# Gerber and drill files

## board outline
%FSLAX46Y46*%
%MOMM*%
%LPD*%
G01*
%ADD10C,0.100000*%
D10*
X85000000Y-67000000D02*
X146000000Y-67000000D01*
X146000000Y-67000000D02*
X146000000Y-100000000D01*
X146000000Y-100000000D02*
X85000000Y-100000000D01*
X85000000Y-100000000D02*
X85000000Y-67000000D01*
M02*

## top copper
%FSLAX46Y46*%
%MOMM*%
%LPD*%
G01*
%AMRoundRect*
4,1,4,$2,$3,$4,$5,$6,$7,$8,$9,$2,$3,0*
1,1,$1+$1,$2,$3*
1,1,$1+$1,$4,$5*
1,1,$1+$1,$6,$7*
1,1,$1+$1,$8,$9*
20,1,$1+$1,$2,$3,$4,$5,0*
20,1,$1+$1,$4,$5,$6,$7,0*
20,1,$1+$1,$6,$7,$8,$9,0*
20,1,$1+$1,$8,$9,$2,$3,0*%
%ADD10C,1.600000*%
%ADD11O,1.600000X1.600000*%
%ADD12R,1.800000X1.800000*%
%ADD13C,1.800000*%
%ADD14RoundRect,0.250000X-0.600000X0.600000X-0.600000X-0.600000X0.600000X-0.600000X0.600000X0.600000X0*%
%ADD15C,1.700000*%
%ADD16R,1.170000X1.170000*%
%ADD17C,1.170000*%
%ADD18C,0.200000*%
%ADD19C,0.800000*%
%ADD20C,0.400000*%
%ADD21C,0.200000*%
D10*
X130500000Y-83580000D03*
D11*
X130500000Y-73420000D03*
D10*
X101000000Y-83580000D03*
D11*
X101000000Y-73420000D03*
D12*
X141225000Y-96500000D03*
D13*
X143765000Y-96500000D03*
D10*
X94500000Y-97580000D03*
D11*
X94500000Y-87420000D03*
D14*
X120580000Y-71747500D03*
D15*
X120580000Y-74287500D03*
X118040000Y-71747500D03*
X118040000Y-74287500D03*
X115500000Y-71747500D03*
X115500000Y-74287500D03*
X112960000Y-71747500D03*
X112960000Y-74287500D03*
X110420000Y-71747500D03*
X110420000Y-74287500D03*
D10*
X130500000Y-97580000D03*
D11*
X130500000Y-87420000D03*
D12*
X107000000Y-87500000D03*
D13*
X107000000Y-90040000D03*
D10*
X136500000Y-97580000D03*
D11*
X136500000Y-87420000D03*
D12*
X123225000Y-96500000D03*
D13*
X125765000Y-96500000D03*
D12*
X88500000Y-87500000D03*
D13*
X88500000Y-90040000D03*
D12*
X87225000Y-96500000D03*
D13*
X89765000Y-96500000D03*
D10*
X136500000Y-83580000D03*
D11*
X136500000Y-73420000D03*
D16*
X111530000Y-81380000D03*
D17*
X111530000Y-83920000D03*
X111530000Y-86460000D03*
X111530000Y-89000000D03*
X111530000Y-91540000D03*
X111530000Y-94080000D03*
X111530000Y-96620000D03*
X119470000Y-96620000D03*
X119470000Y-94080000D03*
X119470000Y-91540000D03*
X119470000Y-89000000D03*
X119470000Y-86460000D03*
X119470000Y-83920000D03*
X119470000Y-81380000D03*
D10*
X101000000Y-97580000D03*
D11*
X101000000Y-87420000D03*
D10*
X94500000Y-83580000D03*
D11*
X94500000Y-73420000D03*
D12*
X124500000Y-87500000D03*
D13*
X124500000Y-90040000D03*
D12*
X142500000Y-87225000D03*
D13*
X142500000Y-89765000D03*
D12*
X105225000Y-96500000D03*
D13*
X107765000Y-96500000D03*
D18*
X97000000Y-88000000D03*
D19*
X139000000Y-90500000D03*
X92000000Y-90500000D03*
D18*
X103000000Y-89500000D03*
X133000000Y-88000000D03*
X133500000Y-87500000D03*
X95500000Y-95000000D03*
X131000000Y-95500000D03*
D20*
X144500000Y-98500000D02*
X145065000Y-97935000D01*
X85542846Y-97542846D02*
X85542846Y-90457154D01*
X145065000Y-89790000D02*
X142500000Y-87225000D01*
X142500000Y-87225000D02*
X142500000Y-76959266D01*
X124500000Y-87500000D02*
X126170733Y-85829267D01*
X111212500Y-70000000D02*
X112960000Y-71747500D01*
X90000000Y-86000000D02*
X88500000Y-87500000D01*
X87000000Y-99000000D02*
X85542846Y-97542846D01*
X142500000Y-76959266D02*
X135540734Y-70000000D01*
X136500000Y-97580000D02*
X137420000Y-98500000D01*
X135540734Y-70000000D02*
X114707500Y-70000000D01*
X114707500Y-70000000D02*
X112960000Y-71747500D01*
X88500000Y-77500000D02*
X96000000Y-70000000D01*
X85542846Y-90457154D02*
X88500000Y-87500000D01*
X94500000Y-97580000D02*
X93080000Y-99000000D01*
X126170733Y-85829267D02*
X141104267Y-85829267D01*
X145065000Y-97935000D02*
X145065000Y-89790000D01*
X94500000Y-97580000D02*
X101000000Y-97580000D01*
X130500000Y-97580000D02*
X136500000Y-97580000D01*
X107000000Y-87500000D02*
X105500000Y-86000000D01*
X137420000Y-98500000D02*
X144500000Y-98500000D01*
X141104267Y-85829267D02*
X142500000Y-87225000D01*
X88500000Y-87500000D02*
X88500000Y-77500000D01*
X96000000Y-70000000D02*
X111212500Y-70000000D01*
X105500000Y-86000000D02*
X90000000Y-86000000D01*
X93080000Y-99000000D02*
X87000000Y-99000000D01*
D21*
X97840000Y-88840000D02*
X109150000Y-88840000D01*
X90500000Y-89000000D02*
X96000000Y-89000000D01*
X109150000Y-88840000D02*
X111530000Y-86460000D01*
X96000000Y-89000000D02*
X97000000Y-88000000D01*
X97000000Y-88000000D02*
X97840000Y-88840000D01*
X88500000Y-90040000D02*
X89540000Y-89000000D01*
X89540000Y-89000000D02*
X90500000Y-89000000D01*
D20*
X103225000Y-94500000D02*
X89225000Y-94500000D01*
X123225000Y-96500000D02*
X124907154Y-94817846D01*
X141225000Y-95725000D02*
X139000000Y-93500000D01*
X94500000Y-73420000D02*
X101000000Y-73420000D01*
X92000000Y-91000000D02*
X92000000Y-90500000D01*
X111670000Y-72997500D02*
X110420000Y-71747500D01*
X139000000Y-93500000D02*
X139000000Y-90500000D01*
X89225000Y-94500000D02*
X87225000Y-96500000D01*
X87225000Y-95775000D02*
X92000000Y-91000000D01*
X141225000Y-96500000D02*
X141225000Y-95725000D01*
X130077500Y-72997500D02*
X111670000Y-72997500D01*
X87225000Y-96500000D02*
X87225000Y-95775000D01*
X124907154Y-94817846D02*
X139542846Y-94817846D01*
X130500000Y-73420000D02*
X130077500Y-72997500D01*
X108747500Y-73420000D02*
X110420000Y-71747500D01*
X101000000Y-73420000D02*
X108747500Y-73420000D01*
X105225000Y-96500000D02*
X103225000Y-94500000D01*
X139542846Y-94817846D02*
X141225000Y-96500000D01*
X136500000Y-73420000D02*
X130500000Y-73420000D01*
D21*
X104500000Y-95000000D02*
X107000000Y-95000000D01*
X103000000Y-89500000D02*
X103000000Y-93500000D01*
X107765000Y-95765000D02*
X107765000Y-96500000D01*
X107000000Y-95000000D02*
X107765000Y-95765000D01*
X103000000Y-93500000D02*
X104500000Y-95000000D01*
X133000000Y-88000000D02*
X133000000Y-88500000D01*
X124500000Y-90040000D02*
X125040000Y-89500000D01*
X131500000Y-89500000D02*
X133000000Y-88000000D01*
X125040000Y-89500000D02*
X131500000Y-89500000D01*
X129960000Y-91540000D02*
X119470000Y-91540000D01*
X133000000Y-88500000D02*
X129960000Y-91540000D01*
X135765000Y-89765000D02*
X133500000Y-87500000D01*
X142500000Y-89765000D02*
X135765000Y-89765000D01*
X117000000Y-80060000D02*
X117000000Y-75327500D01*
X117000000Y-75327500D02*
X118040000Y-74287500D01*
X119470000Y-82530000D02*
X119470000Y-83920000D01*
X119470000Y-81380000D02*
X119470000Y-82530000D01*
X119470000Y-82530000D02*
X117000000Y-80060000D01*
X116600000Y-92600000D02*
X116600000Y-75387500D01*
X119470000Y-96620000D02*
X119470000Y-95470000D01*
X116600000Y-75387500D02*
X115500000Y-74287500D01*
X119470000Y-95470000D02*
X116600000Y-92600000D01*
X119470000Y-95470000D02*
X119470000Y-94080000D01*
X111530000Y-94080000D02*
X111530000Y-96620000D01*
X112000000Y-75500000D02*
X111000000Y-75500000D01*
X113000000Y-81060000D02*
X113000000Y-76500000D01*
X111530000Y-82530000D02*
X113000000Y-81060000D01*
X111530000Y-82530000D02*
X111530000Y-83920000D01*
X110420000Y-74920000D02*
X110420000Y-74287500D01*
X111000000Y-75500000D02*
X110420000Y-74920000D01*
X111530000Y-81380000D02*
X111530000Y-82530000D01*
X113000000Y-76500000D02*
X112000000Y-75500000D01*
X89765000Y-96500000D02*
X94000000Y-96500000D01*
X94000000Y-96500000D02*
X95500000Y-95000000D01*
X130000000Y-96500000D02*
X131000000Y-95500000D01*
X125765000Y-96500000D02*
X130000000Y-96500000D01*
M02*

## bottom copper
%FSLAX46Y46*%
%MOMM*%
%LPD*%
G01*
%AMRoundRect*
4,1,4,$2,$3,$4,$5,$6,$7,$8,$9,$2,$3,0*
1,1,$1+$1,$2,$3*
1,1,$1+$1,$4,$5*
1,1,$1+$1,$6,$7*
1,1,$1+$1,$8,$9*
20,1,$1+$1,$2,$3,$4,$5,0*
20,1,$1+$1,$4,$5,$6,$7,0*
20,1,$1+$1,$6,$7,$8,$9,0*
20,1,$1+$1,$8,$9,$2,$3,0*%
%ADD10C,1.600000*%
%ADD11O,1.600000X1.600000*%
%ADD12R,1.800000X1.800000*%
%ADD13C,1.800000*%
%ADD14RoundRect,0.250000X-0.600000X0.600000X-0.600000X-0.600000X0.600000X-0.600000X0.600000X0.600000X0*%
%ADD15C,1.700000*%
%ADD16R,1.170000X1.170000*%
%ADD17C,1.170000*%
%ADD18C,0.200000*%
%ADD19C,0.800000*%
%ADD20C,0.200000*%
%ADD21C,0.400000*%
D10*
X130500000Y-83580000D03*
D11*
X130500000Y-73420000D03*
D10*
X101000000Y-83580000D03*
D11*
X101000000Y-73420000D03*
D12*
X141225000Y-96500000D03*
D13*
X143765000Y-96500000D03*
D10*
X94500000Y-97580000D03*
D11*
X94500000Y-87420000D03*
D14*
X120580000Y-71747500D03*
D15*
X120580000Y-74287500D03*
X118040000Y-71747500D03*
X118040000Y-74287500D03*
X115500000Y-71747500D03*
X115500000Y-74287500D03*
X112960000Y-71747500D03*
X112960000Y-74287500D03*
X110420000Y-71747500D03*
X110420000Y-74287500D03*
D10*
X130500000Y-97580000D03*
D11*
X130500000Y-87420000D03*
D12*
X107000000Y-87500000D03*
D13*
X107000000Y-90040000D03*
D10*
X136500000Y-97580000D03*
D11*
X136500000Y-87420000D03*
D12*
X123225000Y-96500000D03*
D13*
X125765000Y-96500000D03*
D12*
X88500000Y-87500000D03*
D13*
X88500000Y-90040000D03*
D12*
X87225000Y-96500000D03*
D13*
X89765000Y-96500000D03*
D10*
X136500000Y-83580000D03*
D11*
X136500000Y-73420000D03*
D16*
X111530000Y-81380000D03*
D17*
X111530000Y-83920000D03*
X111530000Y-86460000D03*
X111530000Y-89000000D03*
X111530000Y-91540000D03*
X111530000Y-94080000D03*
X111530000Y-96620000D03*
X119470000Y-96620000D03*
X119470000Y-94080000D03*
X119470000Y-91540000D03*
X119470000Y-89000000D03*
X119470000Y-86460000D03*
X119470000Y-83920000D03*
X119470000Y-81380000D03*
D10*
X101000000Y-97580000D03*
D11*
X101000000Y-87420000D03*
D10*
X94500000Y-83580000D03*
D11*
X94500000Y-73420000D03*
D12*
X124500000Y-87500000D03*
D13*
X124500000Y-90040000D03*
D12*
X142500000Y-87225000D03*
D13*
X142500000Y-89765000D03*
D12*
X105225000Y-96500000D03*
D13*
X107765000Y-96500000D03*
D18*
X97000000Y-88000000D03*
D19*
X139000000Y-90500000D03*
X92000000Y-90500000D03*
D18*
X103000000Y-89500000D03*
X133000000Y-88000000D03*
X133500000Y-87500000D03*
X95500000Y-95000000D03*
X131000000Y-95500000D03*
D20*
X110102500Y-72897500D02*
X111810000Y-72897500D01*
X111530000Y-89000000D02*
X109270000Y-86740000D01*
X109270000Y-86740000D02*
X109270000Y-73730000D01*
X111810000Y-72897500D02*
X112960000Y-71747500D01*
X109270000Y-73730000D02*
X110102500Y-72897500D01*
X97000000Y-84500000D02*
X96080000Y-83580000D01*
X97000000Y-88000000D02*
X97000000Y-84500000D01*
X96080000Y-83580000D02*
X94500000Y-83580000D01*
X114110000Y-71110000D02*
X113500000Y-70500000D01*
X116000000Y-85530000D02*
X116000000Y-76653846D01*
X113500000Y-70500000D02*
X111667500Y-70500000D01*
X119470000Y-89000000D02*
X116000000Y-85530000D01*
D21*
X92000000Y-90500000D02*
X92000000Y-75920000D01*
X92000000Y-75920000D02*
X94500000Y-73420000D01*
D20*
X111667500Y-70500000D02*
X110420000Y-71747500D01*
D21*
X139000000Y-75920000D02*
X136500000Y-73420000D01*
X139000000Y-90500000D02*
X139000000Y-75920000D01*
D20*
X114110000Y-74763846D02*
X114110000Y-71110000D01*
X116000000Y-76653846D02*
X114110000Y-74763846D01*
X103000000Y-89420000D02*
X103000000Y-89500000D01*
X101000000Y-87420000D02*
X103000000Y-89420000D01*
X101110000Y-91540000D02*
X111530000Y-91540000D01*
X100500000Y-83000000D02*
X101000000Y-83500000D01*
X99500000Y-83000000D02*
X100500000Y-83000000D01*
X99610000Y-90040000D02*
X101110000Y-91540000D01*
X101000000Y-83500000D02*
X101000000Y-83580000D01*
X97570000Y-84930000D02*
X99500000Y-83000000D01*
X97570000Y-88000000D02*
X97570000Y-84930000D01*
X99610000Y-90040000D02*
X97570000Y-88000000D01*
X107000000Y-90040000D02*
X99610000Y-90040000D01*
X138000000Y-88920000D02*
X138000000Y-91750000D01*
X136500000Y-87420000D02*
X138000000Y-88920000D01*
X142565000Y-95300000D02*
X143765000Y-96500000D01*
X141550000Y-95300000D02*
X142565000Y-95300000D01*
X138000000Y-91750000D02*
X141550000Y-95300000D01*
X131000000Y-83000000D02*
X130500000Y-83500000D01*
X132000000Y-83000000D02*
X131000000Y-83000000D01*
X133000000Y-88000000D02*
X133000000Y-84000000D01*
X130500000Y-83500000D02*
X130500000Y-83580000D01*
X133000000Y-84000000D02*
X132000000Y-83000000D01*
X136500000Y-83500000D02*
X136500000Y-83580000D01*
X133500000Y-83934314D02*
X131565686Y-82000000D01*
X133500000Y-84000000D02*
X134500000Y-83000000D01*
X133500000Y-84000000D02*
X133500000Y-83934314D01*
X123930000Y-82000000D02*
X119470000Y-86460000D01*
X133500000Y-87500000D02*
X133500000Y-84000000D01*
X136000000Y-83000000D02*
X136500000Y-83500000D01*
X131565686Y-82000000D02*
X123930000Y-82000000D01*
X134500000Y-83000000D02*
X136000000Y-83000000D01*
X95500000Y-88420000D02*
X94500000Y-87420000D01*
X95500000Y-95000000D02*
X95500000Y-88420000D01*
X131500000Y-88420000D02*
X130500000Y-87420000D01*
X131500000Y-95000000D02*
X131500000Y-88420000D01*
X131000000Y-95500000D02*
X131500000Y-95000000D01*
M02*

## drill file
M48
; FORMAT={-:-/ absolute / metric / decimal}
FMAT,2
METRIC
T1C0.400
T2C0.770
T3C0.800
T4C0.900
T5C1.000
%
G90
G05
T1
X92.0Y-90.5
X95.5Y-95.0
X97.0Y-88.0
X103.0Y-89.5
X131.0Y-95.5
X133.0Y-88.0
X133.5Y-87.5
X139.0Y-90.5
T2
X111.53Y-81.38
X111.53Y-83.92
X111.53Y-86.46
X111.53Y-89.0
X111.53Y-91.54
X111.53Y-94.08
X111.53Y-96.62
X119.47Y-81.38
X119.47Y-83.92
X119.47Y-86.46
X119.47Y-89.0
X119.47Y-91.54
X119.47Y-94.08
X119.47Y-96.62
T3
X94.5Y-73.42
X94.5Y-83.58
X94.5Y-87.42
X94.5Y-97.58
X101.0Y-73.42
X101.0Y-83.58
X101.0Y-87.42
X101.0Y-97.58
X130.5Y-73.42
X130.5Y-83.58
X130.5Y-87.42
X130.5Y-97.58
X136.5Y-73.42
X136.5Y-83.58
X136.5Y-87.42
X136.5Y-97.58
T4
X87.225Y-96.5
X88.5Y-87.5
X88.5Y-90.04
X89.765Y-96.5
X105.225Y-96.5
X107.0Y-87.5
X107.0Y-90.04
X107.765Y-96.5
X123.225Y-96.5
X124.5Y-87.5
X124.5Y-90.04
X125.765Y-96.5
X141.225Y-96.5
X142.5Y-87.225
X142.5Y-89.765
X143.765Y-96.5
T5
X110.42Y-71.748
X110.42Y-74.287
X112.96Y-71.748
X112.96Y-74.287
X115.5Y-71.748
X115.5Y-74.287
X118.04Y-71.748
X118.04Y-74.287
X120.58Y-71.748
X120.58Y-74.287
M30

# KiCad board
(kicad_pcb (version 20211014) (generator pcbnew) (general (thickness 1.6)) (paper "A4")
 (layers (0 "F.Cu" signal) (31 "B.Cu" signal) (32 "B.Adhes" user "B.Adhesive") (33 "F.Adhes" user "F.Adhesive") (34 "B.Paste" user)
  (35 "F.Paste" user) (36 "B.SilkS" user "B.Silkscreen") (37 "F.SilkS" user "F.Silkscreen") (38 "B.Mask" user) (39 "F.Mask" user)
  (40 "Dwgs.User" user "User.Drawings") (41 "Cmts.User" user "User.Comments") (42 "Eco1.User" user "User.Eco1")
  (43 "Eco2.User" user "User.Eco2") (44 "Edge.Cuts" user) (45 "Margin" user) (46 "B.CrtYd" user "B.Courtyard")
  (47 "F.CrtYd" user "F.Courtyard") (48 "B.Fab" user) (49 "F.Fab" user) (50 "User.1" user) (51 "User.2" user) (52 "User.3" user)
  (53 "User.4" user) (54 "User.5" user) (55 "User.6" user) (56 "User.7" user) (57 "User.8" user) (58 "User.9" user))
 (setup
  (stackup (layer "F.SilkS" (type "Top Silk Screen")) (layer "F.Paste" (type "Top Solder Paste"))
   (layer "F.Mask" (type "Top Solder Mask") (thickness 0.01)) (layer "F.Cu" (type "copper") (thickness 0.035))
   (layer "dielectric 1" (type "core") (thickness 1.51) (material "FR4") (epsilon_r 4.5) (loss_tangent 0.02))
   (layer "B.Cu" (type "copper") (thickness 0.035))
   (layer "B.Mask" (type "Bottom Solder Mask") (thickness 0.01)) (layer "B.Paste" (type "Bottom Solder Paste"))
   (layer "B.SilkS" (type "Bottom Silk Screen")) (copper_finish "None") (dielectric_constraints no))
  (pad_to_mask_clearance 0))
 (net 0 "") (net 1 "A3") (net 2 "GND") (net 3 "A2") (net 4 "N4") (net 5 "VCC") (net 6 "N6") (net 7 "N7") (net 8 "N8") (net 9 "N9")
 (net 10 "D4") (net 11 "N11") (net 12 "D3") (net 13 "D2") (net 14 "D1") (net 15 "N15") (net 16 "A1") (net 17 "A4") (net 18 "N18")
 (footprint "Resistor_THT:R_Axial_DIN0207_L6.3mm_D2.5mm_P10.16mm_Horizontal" (layer "F.Cu") (at 130.5 83.58 90)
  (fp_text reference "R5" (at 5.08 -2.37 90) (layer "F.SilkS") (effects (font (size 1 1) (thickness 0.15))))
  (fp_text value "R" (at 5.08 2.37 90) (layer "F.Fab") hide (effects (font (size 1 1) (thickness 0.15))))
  (pad "1" thru_hole circle (at 0 0 90) (size 1.6 1.6) (drill 0.8) (layers *.Cu *.Mask) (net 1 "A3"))
  (pad "2" thru_hole oval (at 10.16 0 90) (size 1.6 1.6) (drill 0.8) (layers *.Cu *.Mask) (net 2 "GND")))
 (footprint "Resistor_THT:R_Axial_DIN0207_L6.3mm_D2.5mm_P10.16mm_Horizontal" (layer "F.Cu") (at 101 83.58 90)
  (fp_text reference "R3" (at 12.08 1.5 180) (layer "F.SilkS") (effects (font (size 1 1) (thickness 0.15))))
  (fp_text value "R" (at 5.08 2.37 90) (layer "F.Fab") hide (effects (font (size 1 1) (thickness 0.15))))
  (pad "1" thru_hole circle (at 0 0 90) (size 1.6 1.6) (drill 0.8) (layers *.Cu *.Mask) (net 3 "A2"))
  (pad "2" thru_hole oval (at 10.16 0 90) (size 1.6 1.6) (drill 0.8) (layers *.Cu *.Mask) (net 2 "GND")))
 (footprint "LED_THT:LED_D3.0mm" (layer "F.Cu") (at 141.225 96.5)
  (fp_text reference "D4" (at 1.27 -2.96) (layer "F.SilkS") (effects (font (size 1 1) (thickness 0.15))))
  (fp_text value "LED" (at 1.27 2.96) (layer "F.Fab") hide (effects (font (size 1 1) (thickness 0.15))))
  (pad "1" thru_hole rect (at 0 0) (size 1.8 1.8) (drill 0.9) (layers *.Cu *.Mask) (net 2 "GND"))
  (pad "2" thru_hole circle (at 2.54 0) (size 1.8 1.8) (drill 0.9) (layers *.Cu *.Mask) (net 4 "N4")))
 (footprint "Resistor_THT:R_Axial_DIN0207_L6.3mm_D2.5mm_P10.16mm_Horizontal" (layer "F.Cu") (at 94.5 97.58 90)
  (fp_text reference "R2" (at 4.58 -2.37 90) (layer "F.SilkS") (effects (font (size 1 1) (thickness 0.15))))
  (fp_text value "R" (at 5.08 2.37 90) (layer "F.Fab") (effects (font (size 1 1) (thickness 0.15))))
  (pad "1" thru_hole circle (at 0 0 90) (size 1.6 1.6) (drill 0.8) (layers *.Cu *.Mask) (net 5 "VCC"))
  (pad "2" thru_hole oval (at 10.16 0 90) (size 1.6 1.6) (drill 0.8) (layers *.Cu *.Mask) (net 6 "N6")))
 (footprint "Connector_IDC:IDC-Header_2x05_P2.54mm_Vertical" (layer "F.Cu") (at 120.58 71.7475 -90)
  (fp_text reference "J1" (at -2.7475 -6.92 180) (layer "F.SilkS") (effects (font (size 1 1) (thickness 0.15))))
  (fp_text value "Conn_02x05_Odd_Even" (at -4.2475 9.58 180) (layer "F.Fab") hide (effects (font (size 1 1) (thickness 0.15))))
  (pad "1" thru_hole roundrect (at 0 0 270) (size 1.7 1.7) (drill 1) (layers *.Cu *.Mask) (roundrect_rratio 0.147059) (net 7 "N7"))
  (pad "2" thru_hole circle (at 2.54 0 270) (size 1.7 1.7) (drill 1) (layers *.Cu *.Mask) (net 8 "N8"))
  (pad "3" thru_hole circle (at 0 2.54 270) (size 1.7 1.7) (drill 1) (layers *.Cu *.Mask) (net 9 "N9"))
  (pad "4" thru_hole circle (at 2.54 2.54 270) (size 1.7 1.7) (drill 1) (layers *.Cu *.Mask) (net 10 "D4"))
  (pad "5" thru_hole circle (at 0 5.08 270) (size 1.7 1.7) (drill 1) (layers *.Cu *.Mask) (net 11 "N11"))
  (pad "6" thru_hole circle (at 2.54 5.08 270) (size 1.7 1.7) (drill 1) (layers *.Cu *.Mask) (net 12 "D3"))
  (pad "7" thru_hole circle (at 0 7.62 270) (size 1.7 1.7) (drill 1) (layers *.Cu *.Mask) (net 5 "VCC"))
  (pad "8" thru_hole circle (at 2.54 7.62 270) (size 1.7 1.7) (drill 1) (layers *.Cu *.Mask) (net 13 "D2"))
  (pad "9" thru_hole circle (at 0 10.16 270) (size 1.7 1.7) (drill 1) (layers *.Cu *.Mask) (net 2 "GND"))
  (pad "10" thru_hole circle (at 2.54 10.16 270) (size 1.7 1.7) (drill 1) (layers *.Cu *.Mask) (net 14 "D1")))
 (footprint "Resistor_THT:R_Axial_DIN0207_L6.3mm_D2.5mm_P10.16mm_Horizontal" (layer "F.Cu") (at 130.5 97.58 90)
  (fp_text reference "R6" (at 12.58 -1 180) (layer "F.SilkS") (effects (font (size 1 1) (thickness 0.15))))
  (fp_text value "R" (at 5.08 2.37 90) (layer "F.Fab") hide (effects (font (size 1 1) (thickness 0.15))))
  (pad "1" thru_hole circle (at 0 0 90) (size 1.6 1.6) (drill 0.8) (layers *.Cu *.Mask) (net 5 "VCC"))
  (pad "2" thru_hole oval (at 10.16 0 90) (size 1.6 1.6) (drill 0.8) (layers *.Cu *.Mask) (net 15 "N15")))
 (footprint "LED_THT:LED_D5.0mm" (layer "F.Cu") (at 107 87.5 -90)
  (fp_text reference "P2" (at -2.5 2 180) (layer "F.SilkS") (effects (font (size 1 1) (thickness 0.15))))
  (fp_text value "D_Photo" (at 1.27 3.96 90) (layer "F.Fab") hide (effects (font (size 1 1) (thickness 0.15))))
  (pad "1" thru_hole rect (at 0 0 270) (size 1.8 1.8) (drill 0.9) (layers *.Cu *.Mask) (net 5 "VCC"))
  (pad "2" thru_hole circle (at 2.54 0 270) (size 1.8 1.8) (drill 0.9) (layers *.Cu *.Mask) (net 3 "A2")))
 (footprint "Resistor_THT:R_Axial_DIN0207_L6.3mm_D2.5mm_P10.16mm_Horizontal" (layer "F.Cu") (at 136.5 97.58 90)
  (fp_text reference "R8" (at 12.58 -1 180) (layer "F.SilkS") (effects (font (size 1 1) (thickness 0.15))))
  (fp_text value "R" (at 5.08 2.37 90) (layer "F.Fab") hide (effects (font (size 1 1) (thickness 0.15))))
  (pad "1" thru_hole circle (at 0 0 90) (size 1.6 1.6) (drill 0.8) (layers *.Cu *.Mask) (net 5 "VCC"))
  (pad "2" thru_hole oval (at 10.16 0 90) (size 1.6 1.6) (drill 0.8) (layers *.Cu *.Mask) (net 4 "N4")))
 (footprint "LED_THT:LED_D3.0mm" (layer "F.Cu") (at 123.225 96.5)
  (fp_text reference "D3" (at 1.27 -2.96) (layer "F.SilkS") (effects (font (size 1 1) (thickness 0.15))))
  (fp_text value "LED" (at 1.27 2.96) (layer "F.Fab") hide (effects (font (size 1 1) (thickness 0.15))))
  (pad "1" thru_hole rect (at 0 0) (size 1.8 1.8) (drill 0.9) (layers *.Cu *.Mask) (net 2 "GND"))
  (pad "2" thru_hole circle (at 2.54 0) (size 1.8 1.8) (drill 0.9) (layers *.Cu *.Mask) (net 15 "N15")))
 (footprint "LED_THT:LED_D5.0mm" (layer "F.Cu") (at 88.5 87.5 -90)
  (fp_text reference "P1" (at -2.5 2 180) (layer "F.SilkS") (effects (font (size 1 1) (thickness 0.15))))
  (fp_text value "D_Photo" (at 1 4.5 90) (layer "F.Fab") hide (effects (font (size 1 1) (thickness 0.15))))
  (pad "1" thru_hole rect (at 0 0 270) (size 1.8 1.8) (drill 0.9) (layers *.Cu *.Mask) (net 5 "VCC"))
  (pad "2" thru_hole circle (at 2.54 0 270) (size 1.8 1.8) (drill 0.9) (layers *.Cu *.Mask) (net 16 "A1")))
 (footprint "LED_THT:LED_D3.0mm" (layer "F.Cu") (at 87.225 96.5)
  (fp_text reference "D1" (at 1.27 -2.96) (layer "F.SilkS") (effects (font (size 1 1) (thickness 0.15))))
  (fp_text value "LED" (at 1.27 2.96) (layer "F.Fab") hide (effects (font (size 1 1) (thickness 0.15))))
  (pad "1" thru_hole rect (at 0 0) (size 1.8 1.8) (drill 0.9) (layers *.Cu *.Mask) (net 2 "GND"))
  (pad "2" thru_hole circle (at 2.54 0) (size 1.8 1.8) (drill 0.9) (layers *.Cu *.Mask) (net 6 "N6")))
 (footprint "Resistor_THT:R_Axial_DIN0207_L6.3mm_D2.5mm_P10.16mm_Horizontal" (layer "F.Cu") (at 136.5 83.58 90)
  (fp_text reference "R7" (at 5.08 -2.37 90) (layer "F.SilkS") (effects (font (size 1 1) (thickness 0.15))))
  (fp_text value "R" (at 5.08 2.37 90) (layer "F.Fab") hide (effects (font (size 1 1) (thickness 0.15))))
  (pad "1" thru_hole circle (at 0 0 90) (size 1.6 1.6) (drill 0.8) (layers *.Cu *.Mask) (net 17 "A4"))
  (pad "2" thru_hole oval (at 10.16 0 90) (size 1.6 1.6) (drill 0.8) (layers *.Cu *.Mask) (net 2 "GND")))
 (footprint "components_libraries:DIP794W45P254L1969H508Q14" (layer "F.Cu") (at 115.5 89)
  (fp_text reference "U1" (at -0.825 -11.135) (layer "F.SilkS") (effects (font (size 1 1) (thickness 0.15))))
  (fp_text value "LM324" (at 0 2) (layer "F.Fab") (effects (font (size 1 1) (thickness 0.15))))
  (pad "1" thru_hole rect locked (at -3.97 -7.62) (size 1.17 1.17) (drill 0.77) (layers *.Cu *.Mask) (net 14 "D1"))
  (pad "2" thru_hole circle locked (at -3.97 -5.08) (size 1.17 1.17) (drill 0.77) (layers *.Cu *.Mask) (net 14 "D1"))
  (pad "3" thru_hole circle locked (at -3.97 -2.54) (size 1.17 1.17) (drill 0.77) (layers *.Cu *.Mask) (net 16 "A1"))
  (pad "4" thru_hole circle locked (at -3.97 0) (size 1.17 1.17) (drill 0.77) (layers *.Cu *.Mask) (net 5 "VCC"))
  (pad "5" thru_hole circle locked (at -3.97 2.54) (size 1.17 1.17) (drill 0.77) (layers *.Cu *.Mask) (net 3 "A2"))
  (pad "6" thru_hole circle locked (at -3.97 5.08) (size 1.17 1.17) (drill 0.77) (layers *.Cu *.Mask) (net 13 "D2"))
  (pad "7" thru_hole circle locked (at -3.97 7.62) (size 1.17 1.17) (drill 0.77) (layers *.Cu *.Mask) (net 13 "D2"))
  (pad "8" thru_hole circle locked (at 3.97 7.62) (size 1.17 1.17) (drill 0.77) (layers *.Cu *.Mask) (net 12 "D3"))
  (pad "9" thru_hole circle locked (at 3.97 5.08) (size 1.17 1.17) (drill 0.77) (layers *.Cu *.Mask) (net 12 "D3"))
  (pad "10" thru_hole circle locked (at 3.97 2.54) (size 1.17 1.17) (drill 0.77) (layers *.Cu *.Mask) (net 1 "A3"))
  (pad "11" thru_hole circle locked (at 3.97 0) (size 1.17 1.17) (drill 0.77) (layers *.Cu *.Mask) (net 2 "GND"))
  (pad "12" thru_hole circle locked (at 3.97 -2.54) (size 1.17 1.17) (drill 0.77) (layers *.Cu *.Mask) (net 17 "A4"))
  (pad "13" thru_hole circle locked (at 3.97 -5.08) (size 1.17 1.17) (drill 0.77) (layers *.Cu *.Mask) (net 10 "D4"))
  (pad "14" thru_hole circle locked (at 3.97 -7.62) (size 1.17 1.17) (drill 0.77) (layers *.Cu *.Mask) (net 10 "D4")))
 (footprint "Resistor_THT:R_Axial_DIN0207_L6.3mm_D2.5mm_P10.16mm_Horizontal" (layer "F.Cu") (at 101 97.58 90)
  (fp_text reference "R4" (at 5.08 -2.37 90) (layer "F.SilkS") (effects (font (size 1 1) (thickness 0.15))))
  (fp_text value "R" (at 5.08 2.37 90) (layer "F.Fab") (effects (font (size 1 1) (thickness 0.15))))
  (pad "1" thru_hole circle (at 0 0 90) (size 1.6 1.6) (drill 0.8) (layers *.Cu *.Mask) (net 5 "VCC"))
  (pad "2" thru_hole oval (at 10.16 0 90) (size 1.6 1.6) (drill 0.8) (layers *.Cu *.Mask) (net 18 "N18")))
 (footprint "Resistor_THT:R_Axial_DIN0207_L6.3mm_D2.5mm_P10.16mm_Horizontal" (layer "F.Cu") (at 94.5 83.58 90)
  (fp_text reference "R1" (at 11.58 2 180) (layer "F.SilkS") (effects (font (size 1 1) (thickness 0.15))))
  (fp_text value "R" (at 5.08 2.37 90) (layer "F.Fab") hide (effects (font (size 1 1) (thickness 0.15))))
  (pad "1" thru_hole circle (at 0 0 90) (size 1.6 1.6) (drill 0.8) (layers *.Cu *.Mask) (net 16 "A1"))
  (pad "2" thru_hole oval (at 10.16 0 90) (size 1.6 1.6) (drill 0.8) (layers *.Cu *.Mask) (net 2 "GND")))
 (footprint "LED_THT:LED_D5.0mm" (layer "F.Cu") (at 124.5 87.5 -90)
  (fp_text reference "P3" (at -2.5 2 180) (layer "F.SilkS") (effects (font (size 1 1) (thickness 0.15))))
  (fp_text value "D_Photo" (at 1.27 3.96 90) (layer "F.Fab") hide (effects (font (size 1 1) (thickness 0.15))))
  (pad "1" thru_hole rect (at 0 0 270) (size 1.8 1.8) (drill 0.9) (layers *.Cu *.Mask) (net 5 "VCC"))
  (pad "2" thru_hole circle (at 2.54 0 270) (size 1.8 1.8) (drill 0.9) (layers *.Cu *.Mask) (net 1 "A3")))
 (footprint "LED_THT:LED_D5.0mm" (layer "F.Cu") (at 142.5 87.225 -90)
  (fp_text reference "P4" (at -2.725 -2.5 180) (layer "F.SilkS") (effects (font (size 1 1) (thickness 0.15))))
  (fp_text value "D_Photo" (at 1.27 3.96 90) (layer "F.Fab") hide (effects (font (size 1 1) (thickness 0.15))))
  (pad "1" thru_hole rect (at 0 0 270) (size 1.8 1.8) (drill 0.9) (layers *.Cu *.Mask) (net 5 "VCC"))
  (pad "2" thru_hole circle (at 2.54 0 270) (size 1.8 1.8) (drill 0.9) (layers *.Cu *.Mask) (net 17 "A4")))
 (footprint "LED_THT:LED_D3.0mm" (layer "F.Cu") (at 105.225 96.5)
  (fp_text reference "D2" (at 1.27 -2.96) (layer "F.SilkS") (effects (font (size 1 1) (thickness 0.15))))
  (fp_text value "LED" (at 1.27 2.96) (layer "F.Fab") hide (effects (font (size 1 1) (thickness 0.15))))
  (pad "1" thru_hole rect (at 0 0) (size 1.8 1.8) (drill 0.9) (layers *.Cu *.Mask) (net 2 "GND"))
  (pad "2" thru_hole circle (at 2.54 0) (size 1.8 1.8) (drill 0.9) (layers *.Cu *.Mask) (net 18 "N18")))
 (gr_line (start 85 67) (end 146 67) (layer "Edge.Cuts") (width 0.1))
 (gr_line (start 146 67) (end 146 100) (layer "Edge.Cuts") (width 0.1))
 (gr_line (start 146 100) (end 85 100) (layer "Edge.Cuts") (width 0.1))
 (gr_line (start 85 100) (end 85 67) (layer "Edge.Cuts") (width 0.1))
 (segment (start 144.5 98.5) (end 145.065 97.935) (width 0.4) (layer "F.Cu") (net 5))
 (segment (start 85.542846 97.542846) (end 85.542846 90.457154) (width 0.4) (layer "F.Cu") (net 5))
 (segment (start 145.065 89.79) (end 142.5 87.225) (width 0.4) (layer "F.Cu") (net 5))
 (segment (start 142.5 87.225) (end 142.5 76.959266) (width 0.4) (layer "F.Cu") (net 5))
 (segment (start 124.5 87.5) (end 126.170733 85.829267) (width 0.4) (layer "F.Cu") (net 5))
 (segment (start 111.2125 70) (end 112.96 71.7475) (width 0.4) (layer "F.Cu") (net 5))
 (segment (start 90 86) (end 88.5 87.5) (width 0.4) (layer "F.Cu") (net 5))
 (segment (start 87 99) (end 85.542846 97.542846) (width 0.4) (layer "F.Cu") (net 5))
 (segment (start 142.5 76.959266) (end 135.540734 70) (width 0.4) (layer "F.Cu") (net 5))
 (segment (start 136.5 97.58) (end 137.42 98.5) (width 0.4) (layer "F.Cu") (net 5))
 (segment (start 135.540734 70) (end 114.7075 70) (width 0.4) (layer "F.Cu") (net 5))
 (segment (start 114.7075 70) (end 112.96 71.7475) (width 0.4) (layer "F.Cu") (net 5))
 (segment (start 88.5 77.5) (end 96 70) (width 0.4) (layer "F.Cu") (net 5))
 (segment (start 85.542846 90.457154) (end 88.5 87.5) (width 0.4) (layer "F.Cu") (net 5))
 (segment (start 94.5 97.58) (end 93.08 99) (width 0.4) (layer "F.Cu") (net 5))
 (segment (start 126.170733 85.829267) (end 141.104267 85.829267) (width 0.4) (layer "F.Cu") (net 5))
 (segment (start 145.065 97.935) (end 145.065 89.79) (width 0.4) (layer "F.Cu") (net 5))
 (segment (start 94.5 97.58) (end 101 97.58) (width 0.4) (layer "F.Cu") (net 5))
 (segment (start 130.5 97.58) (end 136.5 97.58) (width 0.4) (layer "F.Cu") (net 5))
 (segment (start 107 87.5) (end 105.5 86) (width 0.4) (layer "F.Cu") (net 5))
 (segment (start 137.42 98.5) (end 144.5 98.5) (width 0.4) (layer "F.Cu") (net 5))
 (segment (start 141.104267 85.829267) (end 142.5 87.225) (width 0.4) (layer "F.Cu") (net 5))
 (segment (start 88.5 87.5) (end 88.5 77.5) (width 0.4) (layer "F.Cu") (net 5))
 (segment (start 96 70) (end 111.2125 70) (width 0.4) (layer "F.Cu") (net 5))
 (segment (start 105.5 86) (end 90 86) (width 0.4) (layer "F.Cu") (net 5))
 (segment (start 93.08 99) (end 87 99) (width 0.4) (layer "F.Cu") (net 5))
 (segment (start 110.1025 72.8975) (end 111.81 72.8975) (width 0.2) (layer "B.Cu") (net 5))
 (segment (start 111.53 89) (end 109.27 86.74) (width 0.2) (layer "B.Cu") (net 5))
 (segment (start 109.27 86.74) (end 109.27 73.73) (width 0.2) (layer "B.Cu") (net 5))
 (segment (start 111.81 72.8975) (end 112.96 71.7475) (width 0.2) (layer "B.Cu") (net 5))
 (segment (start 109.27 73.73) (end 110.1025 72.8975) (width 0.2) (layer "B.Cu") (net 5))
 (segment (start 97.84 88.84) (end 109.15 88.84) (width 0.2) (layer "F.Cu") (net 16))
 (segment (start 90.5 89) (end 96 89) (width 0.2) (layer "F.Cu") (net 16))
 (segment (start 109.15 88.84) (end 111.53 86.46) (width 0.2) (layer "F.Cu") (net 16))
 (segment (start 96 89) (end 97 88) (width 0.2) (layer "F.Cu") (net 16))
 (segment (start 97 88) (end 97.84 88.84) (width 0.2) (layer "F.Cu") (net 16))
 (segment (start 88.5 90.04) (end 89.54 89) (width 0.2) (layer "F.Cu") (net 16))
 (segment (start 89.54 89) (end 90.5 89) (width 0.2) (layer "F.Cu") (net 16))
 (via (at 97 88) (size 0.2) (drill 0.4) (layers "F.Cu" "B.Cu") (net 16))
 (segment (start 97 84.5) (end 96.08 83.58) (width 0.2) (layer "B.Cu") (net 16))
 (segment (start 97 88) (end 97 84.5) (width 0.2) (layer "B.Cu") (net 16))
 (segment (start 96.08 83.58) (end 94.5 83.58) (width 0.2) (layer "B.Cu") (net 16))
 (segment (start 103.225 94.5) (end 89.225 94.5) (width 0.4) (layer "F.Cu") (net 2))
 (segment (start 123.225 96.5) (end 124.907154 94.817846) (width 0.4) (layer "F.Cu") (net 2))
 (segment (start 141.225 95.725) (end 139 93.5) (width 0.4) (layer "F.Cu") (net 2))
 (segment (start 94.5 73.42) (end 101 73.42) (width 0.4) (layer "F.Cu") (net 2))
 (segment (start 92 91) (end 92 90.5) (width 0.4) (layer "F.Cu") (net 2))
 (segment (start 111.67 72.9975) (end 110.42 71.7475) (width 0.4) (layer "F.Cu") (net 2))
 (segment (start 139 93.5) (end 139 90.5) (width 0.4) (layer "F.Cu") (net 2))
 (segment (start 89.225 94.5) (end 87.225 96.5) (width 0.4) (layer "F.Cu") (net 2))
 (segment (start 87.225 95.775) (end 92 91) (width 0.4) (layer "F.Cu") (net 2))
 (segment (start 141.225 96.5) (end 141.225 95.725) (width 0.4) (layer "F.Cu") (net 2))
 (segment (start 130.0775 72.9975) (end 111.67 72.9975) (width 0.4) (layer "F.Cu") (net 2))
 (segment (start 87.225 96.5) (end 87.225 95.775) (width 0.4) (layer "F.Cu") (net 2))
 (segment (start 124.907154 94.817846) (end 139.542846 94.817846) (width 0.4) (layer "F.Cu") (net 2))
 (segment (start 130.5 73.42) (end 130.0775 72.9975) (width 0.4) (layer "F.Cu") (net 2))
 (segment (start 108.7475 73.42) (end 110.42 71.7475) (width 0.4) (layer "F.Cu") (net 2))
 (segment (start 101 73.42) (end 108.7475 73.42) (width 0.4) (layer "F.Cu") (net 2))
 (segment (start 105.225 96.5) (end 103.225 94.5) (width 0.4) (layer "F.Cu") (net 2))
 (segment (start 139.542846 94.817846) (end 141.225 96.5) (width 0.4) (layer "F.Cu") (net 2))
 (segment (start 136.5 73.42) (end 130.5 73.42) (width 0.4) (layer "F.Cu") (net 2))
 (via (at 139 90.5) (size 0.8) (drill 0.4) (layers "F.Cu" "B.Cu") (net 2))
 (via (at 92 90.5) (size 0.8) (drill 0.4) (layers "F.Cu" "B.Cu") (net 2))
 (segment (start 114.11 71.11) (end 113.5 70.5) (width 0.2) (layer "B.Cu") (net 2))
 (segment (start 116 85.53) (end 116 76.653846) (width 0.2) (layer "B.Cu") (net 2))
 (segment (start 113.5 70.5) (end 111.6675 70.5) (width 0.2) (layer "B.Cu") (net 2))
 (segment (start 119.47 89) (end 116 85.53) (width 0.2) (layer "B.Cu") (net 2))
 (segment (start 92 90.5) (end 92 75.92) (width 0.4) (layer "B.Cu") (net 2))
 (segment (start 92 75.92) (end 94.5 73.42) (width 0.4) (layer "B.Cu") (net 2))
 (segment (start 111.6675 70.5) (end 110.42 71.7475) (width 0.2) (layer "B.Cu") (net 2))
 (segment (start 139 75.92) (end 136.5 73.42) (width 0.4) (layer "B.Cu") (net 2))
 (segment (start 139 90.5) (end 139 75.92) (width 0.4) (layer "B.Cu") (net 2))
 (segment (start 114.11 74.763846) (end 114.11 71.11) (width 0.2) (layer "B.Cu") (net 2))
 (segment (start 116 76.653846) (end 114.11 74.763846) (width 0.2) (layer "B.Cu") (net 2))
 (segment (start 104.5 95) (end 107 95) (width 0.2) (layer "F.Cu") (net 18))
 (segment (start 103 89.5) (end 103 93.5) (width 0.2) (layer "F.Cu") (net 18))
 (segment (start 107.765 95.765) (end 107.765 96.5) (width 0.2) (layer "F.Cu") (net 18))
 (segment (start 107 95) (end 107.765 95.765) (width 0.2) (layer "F.Cu") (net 18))
 (segment (start 103 93.5) (end 104.5 95) (width 0.2) (layer "F.Cu") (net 18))
 (via (at 103 89.5) (size 0.2) (drill 0.4) (layers "F.Cu" "B.Cu") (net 18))
 (segment (start 103 89.42) (end 103 89.5) (width 0.2) (layer "B.Cu") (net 18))
 (segment (start 101 87.42) (end 103 89.42) (width 0.2) (layer "B.Cu") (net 18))
 (segment (start 101.11 91.54) (end 111.53 91.54) (width 0.2) (layer "B.Cu") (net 3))
 (segment (start 100.5 83) (end 101 83.5) (width 0.2) (layer "B.Cu") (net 3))
 (segment (start 99.5 83) (end 100.5 83) (width 0.2) (layer "B.Cu") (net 3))
 (segment (start 99.61 90.04) (end 101.11 91.54) (width 0.2) (layer "B.Cu") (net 3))
 (segment (start 101 83.5) (end 101 83.58) (width 0.2) (layer "B.Cu") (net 3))
 (segment (start 97.57 84.93) (end 99.5 83) (width 0.2) (layer "B.Cu") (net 3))
 (segment (start 97.57 88) (end 97.57 84.93) (width 0.2) (layer "B.Cu") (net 3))
 (segment (start 99.61 90.04) (end 97.57 88) (width 0.2) (layer "B.Cu") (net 3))
 (segment (start 107 90.04) (end 99.61 90.04) (width 0.2) (layer "B.Cu") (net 3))
 (segment (start 138 88.92) (end 138 91.75) (width 0.2) (layer "B.Cu") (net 4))
 (segment (start 136.5 87.42) (end 138 88.92) (width 0.2) (layer "B.Cu") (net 4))
 (segment (start 142.565 95.3) (end 143.765 96.5) (width 0.2) (layer "B.Cu") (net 4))
 (segment (start 141.55 95.3) (end 142.565 95.3) (width 0.2) (layer "B.Cu") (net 4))
 (segment (start 138 91.75) (end 141.55 95.3) (width 0.2) (layer "B.Cu") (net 4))
 (segment (start 133 88) (end 133 88.5) (width 0.2) (layer "F.Cu") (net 1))
 (segment (start 124.5 90.04) (end 125.04 89.5) (width 0.2) (layer "F.Cu") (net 1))
 (segment (start 131.5 89.5) (end 133 88) (width 0.2) (layer "F.Cu") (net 1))
 (segment (start 125.04 89.5) (end 131.5 89.5) (width 0.2) (layer "F.Cu") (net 1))
 (segment (start 129.96 91.54) (end 119.47 91.54) (width 0.2) (layer "F.Cu") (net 1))
 (segment (start 133 88.5) (end 129.96 91.54) (width 0.2) (layer "F.Cu") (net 1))
 (via (at 133 88) (size 0.2) (drill 0.4) (layers "F.Cu" "B.Cu") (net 1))
 (segment (start 131 83) (end 130.5 83.5) (width 0.2) (layer "B.Cu") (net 1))
 (segment (start 132 83) (end 131 83) (width 0.2) (layer "B.Cu") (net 1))
 (segment (start 133 88) (end 133 84) (width 0.2) (layer "B.Cu") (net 1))
 (segment (start 130.5 83.5) (end 130.5 83.58) (width 0.2) (layer "B.Cu") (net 1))
 (segment (start 133 84) (end 132 83) (width 0.2) (layer "B.Cu") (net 1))
 (segment (start 135.765 89.765) (end 133.5 87.5) (width 0.2) (layer "F.Cu") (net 17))
 (segment (start 142.5 89.765) (end 135.765 89.765) (width 0.2) (layer "F.Cu") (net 17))
 (via (at 133.5 87.5) (size 0.2) (drill 0.4) (layers "F.Cu" "B.Cu") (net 17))
 (segment (start 136.5 83.5) (end 136.5 83.58) (width 0.2) (layer "B.Cu") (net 17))
 (segment (start 133.5 83.934314) (end 131.565686 82) (width 0.2) (layer "B.Cu") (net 17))
 (segment (start 133.5 84) (end 134.5 83) (width 0.2) (layer "B.Cu") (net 17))
 (segment (start 133.5 84) (end 133.5 83.934314) (width 0.2) (layer "B.Cu") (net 17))
 (segment (start 123.93 82) (end 119.47 86.46) (width 0.2) (layer "B.Cu") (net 17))
 (segment (start 133.5 87.5) (end 133.5 84) (width 0.2) (layer "B.Cu") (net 17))
 (segment (start 136 83) (end 136.5 83.5) (width 0.2) (layer "B.Cu") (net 17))
 (segment (start 131.565686 82) (end 123.93 82) (width 0.2) (layer "B.Cu") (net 17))
 (segment (start 134.5 83) (end 136 83) (width 0.2) (layer "B.Cu") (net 17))
 (segment (start 117 80.06) (end 117 75.3275) (width 0.2) (layer "F.Cu") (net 10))
 (segment (start 117 75.3275) (end 118.04 74.2875) (width 0.2) (layer "F.Cu") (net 10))
 (segment (start 119.47 82.53) (end 119.47 83.92) (width 0.2) (layer "F.Cu") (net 10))
 (segment (start 119.47 81.38) (end 119.47 82.53) (width 0.2) (layer "F.Cu") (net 10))
 (segment (start 119.47 82.53) (end 117 80.06) (width 0.2) (layer "F.Cu") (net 10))
 (segment (start 116.6 92.6) (end 116.6 75.3875) (width 0.2) (layer "F.Cu") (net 12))
 (segment (start 119.47 96.62) (end 119.47 95.47) (width 0.2) (layer "F.Cu") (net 12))
 (segment (start 116.6 75.3875) (end 115.5 74.2875) (width 0.2) (layer "F.Cu") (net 12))
 (segment (start 119.47 95.47) (end 116.6 92.6) (width 0.2) (layer "F.Cu") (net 12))
 (segment (start 119.47 95.47) (end 119.47 94.08) (width 0.2) (layer "F.Cu") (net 12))
 (segment (start 111.53 94.08) (end 111.53 96.62) (width 0.2) (layer "F.Cu") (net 13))
 (segment (start 112 75.5) (end 111 75.5) (width 0.2) (layer "F.Cu") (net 14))
 (segment (start 113 81.06) (end 113 76.5) (width 0.2) (layer "F.Cu") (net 14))
 (segment (start 111.53 82.53) (end 113 81.06) (width 0.2) (layer "F.Cu") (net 14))
 (segment (start 111.53 82.53) (end 111.53 83.92) (width 0.2) (layer "F.Cu") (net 14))
 (segment (start 110.42 74.92) (end 110.42 74.2875) (width 0.2) (layer "F.Cu") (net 14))
 (segment (start 111 75.5) (end 110.42 74.92) (width 0.2) (layer "F.Cu") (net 14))
 (segment (start 111.53 81.38) (end 111.53 82.53) (width 0.2) (layer "F.Cu") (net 14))
 (segment (start 113 76.5) (end 112 75.5) (width 0.2) (layer "F.Cu") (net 14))
 (segment (start 89.765 96.5) (end 94 96.5) (width 0.2) (layer "F.Cu") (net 6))
 (segment (start 94 96.5) (end 95.5 95) (width 0.2) (layer "F.Cu") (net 6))
 (via (at 95.5 95) (size 0.2) (drill 0.4) (layers "F.Cu" "B.Cu") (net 6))
 (segment (start 95.5 88.42) (end 94.5 87.42) (width 0.2) (layer "B.Cu") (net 6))
 (segment (start 95.5 95) (end 95.5 88.42) (width 0.2) (layer "B.Cu") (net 6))
 (segment (start 130 96.5) (end 131 95.5) (width 0.2) (layer "F.Cu") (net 15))
 (segment (start 125.765 96.5) (end 130 96.5) (width 0.2) (layer "F.Cu") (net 15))
 (via (at 131 95.5) (size 0.2) (drill 0.4) (layers "F.Cu" "B.Cu") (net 15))
 (segment (start 131.5 88.42) (end 130.5 87.42) (width 0.2) (layer "B.Cu") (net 15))
 (segment (start 131.5 95) (end 131.5 88.42) (width 0.2) (layer "B.Cu") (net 15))
 (segment (start 131 95.5) (end 131.5 95) (width 0.2) (layer "B.Cu") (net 15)))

